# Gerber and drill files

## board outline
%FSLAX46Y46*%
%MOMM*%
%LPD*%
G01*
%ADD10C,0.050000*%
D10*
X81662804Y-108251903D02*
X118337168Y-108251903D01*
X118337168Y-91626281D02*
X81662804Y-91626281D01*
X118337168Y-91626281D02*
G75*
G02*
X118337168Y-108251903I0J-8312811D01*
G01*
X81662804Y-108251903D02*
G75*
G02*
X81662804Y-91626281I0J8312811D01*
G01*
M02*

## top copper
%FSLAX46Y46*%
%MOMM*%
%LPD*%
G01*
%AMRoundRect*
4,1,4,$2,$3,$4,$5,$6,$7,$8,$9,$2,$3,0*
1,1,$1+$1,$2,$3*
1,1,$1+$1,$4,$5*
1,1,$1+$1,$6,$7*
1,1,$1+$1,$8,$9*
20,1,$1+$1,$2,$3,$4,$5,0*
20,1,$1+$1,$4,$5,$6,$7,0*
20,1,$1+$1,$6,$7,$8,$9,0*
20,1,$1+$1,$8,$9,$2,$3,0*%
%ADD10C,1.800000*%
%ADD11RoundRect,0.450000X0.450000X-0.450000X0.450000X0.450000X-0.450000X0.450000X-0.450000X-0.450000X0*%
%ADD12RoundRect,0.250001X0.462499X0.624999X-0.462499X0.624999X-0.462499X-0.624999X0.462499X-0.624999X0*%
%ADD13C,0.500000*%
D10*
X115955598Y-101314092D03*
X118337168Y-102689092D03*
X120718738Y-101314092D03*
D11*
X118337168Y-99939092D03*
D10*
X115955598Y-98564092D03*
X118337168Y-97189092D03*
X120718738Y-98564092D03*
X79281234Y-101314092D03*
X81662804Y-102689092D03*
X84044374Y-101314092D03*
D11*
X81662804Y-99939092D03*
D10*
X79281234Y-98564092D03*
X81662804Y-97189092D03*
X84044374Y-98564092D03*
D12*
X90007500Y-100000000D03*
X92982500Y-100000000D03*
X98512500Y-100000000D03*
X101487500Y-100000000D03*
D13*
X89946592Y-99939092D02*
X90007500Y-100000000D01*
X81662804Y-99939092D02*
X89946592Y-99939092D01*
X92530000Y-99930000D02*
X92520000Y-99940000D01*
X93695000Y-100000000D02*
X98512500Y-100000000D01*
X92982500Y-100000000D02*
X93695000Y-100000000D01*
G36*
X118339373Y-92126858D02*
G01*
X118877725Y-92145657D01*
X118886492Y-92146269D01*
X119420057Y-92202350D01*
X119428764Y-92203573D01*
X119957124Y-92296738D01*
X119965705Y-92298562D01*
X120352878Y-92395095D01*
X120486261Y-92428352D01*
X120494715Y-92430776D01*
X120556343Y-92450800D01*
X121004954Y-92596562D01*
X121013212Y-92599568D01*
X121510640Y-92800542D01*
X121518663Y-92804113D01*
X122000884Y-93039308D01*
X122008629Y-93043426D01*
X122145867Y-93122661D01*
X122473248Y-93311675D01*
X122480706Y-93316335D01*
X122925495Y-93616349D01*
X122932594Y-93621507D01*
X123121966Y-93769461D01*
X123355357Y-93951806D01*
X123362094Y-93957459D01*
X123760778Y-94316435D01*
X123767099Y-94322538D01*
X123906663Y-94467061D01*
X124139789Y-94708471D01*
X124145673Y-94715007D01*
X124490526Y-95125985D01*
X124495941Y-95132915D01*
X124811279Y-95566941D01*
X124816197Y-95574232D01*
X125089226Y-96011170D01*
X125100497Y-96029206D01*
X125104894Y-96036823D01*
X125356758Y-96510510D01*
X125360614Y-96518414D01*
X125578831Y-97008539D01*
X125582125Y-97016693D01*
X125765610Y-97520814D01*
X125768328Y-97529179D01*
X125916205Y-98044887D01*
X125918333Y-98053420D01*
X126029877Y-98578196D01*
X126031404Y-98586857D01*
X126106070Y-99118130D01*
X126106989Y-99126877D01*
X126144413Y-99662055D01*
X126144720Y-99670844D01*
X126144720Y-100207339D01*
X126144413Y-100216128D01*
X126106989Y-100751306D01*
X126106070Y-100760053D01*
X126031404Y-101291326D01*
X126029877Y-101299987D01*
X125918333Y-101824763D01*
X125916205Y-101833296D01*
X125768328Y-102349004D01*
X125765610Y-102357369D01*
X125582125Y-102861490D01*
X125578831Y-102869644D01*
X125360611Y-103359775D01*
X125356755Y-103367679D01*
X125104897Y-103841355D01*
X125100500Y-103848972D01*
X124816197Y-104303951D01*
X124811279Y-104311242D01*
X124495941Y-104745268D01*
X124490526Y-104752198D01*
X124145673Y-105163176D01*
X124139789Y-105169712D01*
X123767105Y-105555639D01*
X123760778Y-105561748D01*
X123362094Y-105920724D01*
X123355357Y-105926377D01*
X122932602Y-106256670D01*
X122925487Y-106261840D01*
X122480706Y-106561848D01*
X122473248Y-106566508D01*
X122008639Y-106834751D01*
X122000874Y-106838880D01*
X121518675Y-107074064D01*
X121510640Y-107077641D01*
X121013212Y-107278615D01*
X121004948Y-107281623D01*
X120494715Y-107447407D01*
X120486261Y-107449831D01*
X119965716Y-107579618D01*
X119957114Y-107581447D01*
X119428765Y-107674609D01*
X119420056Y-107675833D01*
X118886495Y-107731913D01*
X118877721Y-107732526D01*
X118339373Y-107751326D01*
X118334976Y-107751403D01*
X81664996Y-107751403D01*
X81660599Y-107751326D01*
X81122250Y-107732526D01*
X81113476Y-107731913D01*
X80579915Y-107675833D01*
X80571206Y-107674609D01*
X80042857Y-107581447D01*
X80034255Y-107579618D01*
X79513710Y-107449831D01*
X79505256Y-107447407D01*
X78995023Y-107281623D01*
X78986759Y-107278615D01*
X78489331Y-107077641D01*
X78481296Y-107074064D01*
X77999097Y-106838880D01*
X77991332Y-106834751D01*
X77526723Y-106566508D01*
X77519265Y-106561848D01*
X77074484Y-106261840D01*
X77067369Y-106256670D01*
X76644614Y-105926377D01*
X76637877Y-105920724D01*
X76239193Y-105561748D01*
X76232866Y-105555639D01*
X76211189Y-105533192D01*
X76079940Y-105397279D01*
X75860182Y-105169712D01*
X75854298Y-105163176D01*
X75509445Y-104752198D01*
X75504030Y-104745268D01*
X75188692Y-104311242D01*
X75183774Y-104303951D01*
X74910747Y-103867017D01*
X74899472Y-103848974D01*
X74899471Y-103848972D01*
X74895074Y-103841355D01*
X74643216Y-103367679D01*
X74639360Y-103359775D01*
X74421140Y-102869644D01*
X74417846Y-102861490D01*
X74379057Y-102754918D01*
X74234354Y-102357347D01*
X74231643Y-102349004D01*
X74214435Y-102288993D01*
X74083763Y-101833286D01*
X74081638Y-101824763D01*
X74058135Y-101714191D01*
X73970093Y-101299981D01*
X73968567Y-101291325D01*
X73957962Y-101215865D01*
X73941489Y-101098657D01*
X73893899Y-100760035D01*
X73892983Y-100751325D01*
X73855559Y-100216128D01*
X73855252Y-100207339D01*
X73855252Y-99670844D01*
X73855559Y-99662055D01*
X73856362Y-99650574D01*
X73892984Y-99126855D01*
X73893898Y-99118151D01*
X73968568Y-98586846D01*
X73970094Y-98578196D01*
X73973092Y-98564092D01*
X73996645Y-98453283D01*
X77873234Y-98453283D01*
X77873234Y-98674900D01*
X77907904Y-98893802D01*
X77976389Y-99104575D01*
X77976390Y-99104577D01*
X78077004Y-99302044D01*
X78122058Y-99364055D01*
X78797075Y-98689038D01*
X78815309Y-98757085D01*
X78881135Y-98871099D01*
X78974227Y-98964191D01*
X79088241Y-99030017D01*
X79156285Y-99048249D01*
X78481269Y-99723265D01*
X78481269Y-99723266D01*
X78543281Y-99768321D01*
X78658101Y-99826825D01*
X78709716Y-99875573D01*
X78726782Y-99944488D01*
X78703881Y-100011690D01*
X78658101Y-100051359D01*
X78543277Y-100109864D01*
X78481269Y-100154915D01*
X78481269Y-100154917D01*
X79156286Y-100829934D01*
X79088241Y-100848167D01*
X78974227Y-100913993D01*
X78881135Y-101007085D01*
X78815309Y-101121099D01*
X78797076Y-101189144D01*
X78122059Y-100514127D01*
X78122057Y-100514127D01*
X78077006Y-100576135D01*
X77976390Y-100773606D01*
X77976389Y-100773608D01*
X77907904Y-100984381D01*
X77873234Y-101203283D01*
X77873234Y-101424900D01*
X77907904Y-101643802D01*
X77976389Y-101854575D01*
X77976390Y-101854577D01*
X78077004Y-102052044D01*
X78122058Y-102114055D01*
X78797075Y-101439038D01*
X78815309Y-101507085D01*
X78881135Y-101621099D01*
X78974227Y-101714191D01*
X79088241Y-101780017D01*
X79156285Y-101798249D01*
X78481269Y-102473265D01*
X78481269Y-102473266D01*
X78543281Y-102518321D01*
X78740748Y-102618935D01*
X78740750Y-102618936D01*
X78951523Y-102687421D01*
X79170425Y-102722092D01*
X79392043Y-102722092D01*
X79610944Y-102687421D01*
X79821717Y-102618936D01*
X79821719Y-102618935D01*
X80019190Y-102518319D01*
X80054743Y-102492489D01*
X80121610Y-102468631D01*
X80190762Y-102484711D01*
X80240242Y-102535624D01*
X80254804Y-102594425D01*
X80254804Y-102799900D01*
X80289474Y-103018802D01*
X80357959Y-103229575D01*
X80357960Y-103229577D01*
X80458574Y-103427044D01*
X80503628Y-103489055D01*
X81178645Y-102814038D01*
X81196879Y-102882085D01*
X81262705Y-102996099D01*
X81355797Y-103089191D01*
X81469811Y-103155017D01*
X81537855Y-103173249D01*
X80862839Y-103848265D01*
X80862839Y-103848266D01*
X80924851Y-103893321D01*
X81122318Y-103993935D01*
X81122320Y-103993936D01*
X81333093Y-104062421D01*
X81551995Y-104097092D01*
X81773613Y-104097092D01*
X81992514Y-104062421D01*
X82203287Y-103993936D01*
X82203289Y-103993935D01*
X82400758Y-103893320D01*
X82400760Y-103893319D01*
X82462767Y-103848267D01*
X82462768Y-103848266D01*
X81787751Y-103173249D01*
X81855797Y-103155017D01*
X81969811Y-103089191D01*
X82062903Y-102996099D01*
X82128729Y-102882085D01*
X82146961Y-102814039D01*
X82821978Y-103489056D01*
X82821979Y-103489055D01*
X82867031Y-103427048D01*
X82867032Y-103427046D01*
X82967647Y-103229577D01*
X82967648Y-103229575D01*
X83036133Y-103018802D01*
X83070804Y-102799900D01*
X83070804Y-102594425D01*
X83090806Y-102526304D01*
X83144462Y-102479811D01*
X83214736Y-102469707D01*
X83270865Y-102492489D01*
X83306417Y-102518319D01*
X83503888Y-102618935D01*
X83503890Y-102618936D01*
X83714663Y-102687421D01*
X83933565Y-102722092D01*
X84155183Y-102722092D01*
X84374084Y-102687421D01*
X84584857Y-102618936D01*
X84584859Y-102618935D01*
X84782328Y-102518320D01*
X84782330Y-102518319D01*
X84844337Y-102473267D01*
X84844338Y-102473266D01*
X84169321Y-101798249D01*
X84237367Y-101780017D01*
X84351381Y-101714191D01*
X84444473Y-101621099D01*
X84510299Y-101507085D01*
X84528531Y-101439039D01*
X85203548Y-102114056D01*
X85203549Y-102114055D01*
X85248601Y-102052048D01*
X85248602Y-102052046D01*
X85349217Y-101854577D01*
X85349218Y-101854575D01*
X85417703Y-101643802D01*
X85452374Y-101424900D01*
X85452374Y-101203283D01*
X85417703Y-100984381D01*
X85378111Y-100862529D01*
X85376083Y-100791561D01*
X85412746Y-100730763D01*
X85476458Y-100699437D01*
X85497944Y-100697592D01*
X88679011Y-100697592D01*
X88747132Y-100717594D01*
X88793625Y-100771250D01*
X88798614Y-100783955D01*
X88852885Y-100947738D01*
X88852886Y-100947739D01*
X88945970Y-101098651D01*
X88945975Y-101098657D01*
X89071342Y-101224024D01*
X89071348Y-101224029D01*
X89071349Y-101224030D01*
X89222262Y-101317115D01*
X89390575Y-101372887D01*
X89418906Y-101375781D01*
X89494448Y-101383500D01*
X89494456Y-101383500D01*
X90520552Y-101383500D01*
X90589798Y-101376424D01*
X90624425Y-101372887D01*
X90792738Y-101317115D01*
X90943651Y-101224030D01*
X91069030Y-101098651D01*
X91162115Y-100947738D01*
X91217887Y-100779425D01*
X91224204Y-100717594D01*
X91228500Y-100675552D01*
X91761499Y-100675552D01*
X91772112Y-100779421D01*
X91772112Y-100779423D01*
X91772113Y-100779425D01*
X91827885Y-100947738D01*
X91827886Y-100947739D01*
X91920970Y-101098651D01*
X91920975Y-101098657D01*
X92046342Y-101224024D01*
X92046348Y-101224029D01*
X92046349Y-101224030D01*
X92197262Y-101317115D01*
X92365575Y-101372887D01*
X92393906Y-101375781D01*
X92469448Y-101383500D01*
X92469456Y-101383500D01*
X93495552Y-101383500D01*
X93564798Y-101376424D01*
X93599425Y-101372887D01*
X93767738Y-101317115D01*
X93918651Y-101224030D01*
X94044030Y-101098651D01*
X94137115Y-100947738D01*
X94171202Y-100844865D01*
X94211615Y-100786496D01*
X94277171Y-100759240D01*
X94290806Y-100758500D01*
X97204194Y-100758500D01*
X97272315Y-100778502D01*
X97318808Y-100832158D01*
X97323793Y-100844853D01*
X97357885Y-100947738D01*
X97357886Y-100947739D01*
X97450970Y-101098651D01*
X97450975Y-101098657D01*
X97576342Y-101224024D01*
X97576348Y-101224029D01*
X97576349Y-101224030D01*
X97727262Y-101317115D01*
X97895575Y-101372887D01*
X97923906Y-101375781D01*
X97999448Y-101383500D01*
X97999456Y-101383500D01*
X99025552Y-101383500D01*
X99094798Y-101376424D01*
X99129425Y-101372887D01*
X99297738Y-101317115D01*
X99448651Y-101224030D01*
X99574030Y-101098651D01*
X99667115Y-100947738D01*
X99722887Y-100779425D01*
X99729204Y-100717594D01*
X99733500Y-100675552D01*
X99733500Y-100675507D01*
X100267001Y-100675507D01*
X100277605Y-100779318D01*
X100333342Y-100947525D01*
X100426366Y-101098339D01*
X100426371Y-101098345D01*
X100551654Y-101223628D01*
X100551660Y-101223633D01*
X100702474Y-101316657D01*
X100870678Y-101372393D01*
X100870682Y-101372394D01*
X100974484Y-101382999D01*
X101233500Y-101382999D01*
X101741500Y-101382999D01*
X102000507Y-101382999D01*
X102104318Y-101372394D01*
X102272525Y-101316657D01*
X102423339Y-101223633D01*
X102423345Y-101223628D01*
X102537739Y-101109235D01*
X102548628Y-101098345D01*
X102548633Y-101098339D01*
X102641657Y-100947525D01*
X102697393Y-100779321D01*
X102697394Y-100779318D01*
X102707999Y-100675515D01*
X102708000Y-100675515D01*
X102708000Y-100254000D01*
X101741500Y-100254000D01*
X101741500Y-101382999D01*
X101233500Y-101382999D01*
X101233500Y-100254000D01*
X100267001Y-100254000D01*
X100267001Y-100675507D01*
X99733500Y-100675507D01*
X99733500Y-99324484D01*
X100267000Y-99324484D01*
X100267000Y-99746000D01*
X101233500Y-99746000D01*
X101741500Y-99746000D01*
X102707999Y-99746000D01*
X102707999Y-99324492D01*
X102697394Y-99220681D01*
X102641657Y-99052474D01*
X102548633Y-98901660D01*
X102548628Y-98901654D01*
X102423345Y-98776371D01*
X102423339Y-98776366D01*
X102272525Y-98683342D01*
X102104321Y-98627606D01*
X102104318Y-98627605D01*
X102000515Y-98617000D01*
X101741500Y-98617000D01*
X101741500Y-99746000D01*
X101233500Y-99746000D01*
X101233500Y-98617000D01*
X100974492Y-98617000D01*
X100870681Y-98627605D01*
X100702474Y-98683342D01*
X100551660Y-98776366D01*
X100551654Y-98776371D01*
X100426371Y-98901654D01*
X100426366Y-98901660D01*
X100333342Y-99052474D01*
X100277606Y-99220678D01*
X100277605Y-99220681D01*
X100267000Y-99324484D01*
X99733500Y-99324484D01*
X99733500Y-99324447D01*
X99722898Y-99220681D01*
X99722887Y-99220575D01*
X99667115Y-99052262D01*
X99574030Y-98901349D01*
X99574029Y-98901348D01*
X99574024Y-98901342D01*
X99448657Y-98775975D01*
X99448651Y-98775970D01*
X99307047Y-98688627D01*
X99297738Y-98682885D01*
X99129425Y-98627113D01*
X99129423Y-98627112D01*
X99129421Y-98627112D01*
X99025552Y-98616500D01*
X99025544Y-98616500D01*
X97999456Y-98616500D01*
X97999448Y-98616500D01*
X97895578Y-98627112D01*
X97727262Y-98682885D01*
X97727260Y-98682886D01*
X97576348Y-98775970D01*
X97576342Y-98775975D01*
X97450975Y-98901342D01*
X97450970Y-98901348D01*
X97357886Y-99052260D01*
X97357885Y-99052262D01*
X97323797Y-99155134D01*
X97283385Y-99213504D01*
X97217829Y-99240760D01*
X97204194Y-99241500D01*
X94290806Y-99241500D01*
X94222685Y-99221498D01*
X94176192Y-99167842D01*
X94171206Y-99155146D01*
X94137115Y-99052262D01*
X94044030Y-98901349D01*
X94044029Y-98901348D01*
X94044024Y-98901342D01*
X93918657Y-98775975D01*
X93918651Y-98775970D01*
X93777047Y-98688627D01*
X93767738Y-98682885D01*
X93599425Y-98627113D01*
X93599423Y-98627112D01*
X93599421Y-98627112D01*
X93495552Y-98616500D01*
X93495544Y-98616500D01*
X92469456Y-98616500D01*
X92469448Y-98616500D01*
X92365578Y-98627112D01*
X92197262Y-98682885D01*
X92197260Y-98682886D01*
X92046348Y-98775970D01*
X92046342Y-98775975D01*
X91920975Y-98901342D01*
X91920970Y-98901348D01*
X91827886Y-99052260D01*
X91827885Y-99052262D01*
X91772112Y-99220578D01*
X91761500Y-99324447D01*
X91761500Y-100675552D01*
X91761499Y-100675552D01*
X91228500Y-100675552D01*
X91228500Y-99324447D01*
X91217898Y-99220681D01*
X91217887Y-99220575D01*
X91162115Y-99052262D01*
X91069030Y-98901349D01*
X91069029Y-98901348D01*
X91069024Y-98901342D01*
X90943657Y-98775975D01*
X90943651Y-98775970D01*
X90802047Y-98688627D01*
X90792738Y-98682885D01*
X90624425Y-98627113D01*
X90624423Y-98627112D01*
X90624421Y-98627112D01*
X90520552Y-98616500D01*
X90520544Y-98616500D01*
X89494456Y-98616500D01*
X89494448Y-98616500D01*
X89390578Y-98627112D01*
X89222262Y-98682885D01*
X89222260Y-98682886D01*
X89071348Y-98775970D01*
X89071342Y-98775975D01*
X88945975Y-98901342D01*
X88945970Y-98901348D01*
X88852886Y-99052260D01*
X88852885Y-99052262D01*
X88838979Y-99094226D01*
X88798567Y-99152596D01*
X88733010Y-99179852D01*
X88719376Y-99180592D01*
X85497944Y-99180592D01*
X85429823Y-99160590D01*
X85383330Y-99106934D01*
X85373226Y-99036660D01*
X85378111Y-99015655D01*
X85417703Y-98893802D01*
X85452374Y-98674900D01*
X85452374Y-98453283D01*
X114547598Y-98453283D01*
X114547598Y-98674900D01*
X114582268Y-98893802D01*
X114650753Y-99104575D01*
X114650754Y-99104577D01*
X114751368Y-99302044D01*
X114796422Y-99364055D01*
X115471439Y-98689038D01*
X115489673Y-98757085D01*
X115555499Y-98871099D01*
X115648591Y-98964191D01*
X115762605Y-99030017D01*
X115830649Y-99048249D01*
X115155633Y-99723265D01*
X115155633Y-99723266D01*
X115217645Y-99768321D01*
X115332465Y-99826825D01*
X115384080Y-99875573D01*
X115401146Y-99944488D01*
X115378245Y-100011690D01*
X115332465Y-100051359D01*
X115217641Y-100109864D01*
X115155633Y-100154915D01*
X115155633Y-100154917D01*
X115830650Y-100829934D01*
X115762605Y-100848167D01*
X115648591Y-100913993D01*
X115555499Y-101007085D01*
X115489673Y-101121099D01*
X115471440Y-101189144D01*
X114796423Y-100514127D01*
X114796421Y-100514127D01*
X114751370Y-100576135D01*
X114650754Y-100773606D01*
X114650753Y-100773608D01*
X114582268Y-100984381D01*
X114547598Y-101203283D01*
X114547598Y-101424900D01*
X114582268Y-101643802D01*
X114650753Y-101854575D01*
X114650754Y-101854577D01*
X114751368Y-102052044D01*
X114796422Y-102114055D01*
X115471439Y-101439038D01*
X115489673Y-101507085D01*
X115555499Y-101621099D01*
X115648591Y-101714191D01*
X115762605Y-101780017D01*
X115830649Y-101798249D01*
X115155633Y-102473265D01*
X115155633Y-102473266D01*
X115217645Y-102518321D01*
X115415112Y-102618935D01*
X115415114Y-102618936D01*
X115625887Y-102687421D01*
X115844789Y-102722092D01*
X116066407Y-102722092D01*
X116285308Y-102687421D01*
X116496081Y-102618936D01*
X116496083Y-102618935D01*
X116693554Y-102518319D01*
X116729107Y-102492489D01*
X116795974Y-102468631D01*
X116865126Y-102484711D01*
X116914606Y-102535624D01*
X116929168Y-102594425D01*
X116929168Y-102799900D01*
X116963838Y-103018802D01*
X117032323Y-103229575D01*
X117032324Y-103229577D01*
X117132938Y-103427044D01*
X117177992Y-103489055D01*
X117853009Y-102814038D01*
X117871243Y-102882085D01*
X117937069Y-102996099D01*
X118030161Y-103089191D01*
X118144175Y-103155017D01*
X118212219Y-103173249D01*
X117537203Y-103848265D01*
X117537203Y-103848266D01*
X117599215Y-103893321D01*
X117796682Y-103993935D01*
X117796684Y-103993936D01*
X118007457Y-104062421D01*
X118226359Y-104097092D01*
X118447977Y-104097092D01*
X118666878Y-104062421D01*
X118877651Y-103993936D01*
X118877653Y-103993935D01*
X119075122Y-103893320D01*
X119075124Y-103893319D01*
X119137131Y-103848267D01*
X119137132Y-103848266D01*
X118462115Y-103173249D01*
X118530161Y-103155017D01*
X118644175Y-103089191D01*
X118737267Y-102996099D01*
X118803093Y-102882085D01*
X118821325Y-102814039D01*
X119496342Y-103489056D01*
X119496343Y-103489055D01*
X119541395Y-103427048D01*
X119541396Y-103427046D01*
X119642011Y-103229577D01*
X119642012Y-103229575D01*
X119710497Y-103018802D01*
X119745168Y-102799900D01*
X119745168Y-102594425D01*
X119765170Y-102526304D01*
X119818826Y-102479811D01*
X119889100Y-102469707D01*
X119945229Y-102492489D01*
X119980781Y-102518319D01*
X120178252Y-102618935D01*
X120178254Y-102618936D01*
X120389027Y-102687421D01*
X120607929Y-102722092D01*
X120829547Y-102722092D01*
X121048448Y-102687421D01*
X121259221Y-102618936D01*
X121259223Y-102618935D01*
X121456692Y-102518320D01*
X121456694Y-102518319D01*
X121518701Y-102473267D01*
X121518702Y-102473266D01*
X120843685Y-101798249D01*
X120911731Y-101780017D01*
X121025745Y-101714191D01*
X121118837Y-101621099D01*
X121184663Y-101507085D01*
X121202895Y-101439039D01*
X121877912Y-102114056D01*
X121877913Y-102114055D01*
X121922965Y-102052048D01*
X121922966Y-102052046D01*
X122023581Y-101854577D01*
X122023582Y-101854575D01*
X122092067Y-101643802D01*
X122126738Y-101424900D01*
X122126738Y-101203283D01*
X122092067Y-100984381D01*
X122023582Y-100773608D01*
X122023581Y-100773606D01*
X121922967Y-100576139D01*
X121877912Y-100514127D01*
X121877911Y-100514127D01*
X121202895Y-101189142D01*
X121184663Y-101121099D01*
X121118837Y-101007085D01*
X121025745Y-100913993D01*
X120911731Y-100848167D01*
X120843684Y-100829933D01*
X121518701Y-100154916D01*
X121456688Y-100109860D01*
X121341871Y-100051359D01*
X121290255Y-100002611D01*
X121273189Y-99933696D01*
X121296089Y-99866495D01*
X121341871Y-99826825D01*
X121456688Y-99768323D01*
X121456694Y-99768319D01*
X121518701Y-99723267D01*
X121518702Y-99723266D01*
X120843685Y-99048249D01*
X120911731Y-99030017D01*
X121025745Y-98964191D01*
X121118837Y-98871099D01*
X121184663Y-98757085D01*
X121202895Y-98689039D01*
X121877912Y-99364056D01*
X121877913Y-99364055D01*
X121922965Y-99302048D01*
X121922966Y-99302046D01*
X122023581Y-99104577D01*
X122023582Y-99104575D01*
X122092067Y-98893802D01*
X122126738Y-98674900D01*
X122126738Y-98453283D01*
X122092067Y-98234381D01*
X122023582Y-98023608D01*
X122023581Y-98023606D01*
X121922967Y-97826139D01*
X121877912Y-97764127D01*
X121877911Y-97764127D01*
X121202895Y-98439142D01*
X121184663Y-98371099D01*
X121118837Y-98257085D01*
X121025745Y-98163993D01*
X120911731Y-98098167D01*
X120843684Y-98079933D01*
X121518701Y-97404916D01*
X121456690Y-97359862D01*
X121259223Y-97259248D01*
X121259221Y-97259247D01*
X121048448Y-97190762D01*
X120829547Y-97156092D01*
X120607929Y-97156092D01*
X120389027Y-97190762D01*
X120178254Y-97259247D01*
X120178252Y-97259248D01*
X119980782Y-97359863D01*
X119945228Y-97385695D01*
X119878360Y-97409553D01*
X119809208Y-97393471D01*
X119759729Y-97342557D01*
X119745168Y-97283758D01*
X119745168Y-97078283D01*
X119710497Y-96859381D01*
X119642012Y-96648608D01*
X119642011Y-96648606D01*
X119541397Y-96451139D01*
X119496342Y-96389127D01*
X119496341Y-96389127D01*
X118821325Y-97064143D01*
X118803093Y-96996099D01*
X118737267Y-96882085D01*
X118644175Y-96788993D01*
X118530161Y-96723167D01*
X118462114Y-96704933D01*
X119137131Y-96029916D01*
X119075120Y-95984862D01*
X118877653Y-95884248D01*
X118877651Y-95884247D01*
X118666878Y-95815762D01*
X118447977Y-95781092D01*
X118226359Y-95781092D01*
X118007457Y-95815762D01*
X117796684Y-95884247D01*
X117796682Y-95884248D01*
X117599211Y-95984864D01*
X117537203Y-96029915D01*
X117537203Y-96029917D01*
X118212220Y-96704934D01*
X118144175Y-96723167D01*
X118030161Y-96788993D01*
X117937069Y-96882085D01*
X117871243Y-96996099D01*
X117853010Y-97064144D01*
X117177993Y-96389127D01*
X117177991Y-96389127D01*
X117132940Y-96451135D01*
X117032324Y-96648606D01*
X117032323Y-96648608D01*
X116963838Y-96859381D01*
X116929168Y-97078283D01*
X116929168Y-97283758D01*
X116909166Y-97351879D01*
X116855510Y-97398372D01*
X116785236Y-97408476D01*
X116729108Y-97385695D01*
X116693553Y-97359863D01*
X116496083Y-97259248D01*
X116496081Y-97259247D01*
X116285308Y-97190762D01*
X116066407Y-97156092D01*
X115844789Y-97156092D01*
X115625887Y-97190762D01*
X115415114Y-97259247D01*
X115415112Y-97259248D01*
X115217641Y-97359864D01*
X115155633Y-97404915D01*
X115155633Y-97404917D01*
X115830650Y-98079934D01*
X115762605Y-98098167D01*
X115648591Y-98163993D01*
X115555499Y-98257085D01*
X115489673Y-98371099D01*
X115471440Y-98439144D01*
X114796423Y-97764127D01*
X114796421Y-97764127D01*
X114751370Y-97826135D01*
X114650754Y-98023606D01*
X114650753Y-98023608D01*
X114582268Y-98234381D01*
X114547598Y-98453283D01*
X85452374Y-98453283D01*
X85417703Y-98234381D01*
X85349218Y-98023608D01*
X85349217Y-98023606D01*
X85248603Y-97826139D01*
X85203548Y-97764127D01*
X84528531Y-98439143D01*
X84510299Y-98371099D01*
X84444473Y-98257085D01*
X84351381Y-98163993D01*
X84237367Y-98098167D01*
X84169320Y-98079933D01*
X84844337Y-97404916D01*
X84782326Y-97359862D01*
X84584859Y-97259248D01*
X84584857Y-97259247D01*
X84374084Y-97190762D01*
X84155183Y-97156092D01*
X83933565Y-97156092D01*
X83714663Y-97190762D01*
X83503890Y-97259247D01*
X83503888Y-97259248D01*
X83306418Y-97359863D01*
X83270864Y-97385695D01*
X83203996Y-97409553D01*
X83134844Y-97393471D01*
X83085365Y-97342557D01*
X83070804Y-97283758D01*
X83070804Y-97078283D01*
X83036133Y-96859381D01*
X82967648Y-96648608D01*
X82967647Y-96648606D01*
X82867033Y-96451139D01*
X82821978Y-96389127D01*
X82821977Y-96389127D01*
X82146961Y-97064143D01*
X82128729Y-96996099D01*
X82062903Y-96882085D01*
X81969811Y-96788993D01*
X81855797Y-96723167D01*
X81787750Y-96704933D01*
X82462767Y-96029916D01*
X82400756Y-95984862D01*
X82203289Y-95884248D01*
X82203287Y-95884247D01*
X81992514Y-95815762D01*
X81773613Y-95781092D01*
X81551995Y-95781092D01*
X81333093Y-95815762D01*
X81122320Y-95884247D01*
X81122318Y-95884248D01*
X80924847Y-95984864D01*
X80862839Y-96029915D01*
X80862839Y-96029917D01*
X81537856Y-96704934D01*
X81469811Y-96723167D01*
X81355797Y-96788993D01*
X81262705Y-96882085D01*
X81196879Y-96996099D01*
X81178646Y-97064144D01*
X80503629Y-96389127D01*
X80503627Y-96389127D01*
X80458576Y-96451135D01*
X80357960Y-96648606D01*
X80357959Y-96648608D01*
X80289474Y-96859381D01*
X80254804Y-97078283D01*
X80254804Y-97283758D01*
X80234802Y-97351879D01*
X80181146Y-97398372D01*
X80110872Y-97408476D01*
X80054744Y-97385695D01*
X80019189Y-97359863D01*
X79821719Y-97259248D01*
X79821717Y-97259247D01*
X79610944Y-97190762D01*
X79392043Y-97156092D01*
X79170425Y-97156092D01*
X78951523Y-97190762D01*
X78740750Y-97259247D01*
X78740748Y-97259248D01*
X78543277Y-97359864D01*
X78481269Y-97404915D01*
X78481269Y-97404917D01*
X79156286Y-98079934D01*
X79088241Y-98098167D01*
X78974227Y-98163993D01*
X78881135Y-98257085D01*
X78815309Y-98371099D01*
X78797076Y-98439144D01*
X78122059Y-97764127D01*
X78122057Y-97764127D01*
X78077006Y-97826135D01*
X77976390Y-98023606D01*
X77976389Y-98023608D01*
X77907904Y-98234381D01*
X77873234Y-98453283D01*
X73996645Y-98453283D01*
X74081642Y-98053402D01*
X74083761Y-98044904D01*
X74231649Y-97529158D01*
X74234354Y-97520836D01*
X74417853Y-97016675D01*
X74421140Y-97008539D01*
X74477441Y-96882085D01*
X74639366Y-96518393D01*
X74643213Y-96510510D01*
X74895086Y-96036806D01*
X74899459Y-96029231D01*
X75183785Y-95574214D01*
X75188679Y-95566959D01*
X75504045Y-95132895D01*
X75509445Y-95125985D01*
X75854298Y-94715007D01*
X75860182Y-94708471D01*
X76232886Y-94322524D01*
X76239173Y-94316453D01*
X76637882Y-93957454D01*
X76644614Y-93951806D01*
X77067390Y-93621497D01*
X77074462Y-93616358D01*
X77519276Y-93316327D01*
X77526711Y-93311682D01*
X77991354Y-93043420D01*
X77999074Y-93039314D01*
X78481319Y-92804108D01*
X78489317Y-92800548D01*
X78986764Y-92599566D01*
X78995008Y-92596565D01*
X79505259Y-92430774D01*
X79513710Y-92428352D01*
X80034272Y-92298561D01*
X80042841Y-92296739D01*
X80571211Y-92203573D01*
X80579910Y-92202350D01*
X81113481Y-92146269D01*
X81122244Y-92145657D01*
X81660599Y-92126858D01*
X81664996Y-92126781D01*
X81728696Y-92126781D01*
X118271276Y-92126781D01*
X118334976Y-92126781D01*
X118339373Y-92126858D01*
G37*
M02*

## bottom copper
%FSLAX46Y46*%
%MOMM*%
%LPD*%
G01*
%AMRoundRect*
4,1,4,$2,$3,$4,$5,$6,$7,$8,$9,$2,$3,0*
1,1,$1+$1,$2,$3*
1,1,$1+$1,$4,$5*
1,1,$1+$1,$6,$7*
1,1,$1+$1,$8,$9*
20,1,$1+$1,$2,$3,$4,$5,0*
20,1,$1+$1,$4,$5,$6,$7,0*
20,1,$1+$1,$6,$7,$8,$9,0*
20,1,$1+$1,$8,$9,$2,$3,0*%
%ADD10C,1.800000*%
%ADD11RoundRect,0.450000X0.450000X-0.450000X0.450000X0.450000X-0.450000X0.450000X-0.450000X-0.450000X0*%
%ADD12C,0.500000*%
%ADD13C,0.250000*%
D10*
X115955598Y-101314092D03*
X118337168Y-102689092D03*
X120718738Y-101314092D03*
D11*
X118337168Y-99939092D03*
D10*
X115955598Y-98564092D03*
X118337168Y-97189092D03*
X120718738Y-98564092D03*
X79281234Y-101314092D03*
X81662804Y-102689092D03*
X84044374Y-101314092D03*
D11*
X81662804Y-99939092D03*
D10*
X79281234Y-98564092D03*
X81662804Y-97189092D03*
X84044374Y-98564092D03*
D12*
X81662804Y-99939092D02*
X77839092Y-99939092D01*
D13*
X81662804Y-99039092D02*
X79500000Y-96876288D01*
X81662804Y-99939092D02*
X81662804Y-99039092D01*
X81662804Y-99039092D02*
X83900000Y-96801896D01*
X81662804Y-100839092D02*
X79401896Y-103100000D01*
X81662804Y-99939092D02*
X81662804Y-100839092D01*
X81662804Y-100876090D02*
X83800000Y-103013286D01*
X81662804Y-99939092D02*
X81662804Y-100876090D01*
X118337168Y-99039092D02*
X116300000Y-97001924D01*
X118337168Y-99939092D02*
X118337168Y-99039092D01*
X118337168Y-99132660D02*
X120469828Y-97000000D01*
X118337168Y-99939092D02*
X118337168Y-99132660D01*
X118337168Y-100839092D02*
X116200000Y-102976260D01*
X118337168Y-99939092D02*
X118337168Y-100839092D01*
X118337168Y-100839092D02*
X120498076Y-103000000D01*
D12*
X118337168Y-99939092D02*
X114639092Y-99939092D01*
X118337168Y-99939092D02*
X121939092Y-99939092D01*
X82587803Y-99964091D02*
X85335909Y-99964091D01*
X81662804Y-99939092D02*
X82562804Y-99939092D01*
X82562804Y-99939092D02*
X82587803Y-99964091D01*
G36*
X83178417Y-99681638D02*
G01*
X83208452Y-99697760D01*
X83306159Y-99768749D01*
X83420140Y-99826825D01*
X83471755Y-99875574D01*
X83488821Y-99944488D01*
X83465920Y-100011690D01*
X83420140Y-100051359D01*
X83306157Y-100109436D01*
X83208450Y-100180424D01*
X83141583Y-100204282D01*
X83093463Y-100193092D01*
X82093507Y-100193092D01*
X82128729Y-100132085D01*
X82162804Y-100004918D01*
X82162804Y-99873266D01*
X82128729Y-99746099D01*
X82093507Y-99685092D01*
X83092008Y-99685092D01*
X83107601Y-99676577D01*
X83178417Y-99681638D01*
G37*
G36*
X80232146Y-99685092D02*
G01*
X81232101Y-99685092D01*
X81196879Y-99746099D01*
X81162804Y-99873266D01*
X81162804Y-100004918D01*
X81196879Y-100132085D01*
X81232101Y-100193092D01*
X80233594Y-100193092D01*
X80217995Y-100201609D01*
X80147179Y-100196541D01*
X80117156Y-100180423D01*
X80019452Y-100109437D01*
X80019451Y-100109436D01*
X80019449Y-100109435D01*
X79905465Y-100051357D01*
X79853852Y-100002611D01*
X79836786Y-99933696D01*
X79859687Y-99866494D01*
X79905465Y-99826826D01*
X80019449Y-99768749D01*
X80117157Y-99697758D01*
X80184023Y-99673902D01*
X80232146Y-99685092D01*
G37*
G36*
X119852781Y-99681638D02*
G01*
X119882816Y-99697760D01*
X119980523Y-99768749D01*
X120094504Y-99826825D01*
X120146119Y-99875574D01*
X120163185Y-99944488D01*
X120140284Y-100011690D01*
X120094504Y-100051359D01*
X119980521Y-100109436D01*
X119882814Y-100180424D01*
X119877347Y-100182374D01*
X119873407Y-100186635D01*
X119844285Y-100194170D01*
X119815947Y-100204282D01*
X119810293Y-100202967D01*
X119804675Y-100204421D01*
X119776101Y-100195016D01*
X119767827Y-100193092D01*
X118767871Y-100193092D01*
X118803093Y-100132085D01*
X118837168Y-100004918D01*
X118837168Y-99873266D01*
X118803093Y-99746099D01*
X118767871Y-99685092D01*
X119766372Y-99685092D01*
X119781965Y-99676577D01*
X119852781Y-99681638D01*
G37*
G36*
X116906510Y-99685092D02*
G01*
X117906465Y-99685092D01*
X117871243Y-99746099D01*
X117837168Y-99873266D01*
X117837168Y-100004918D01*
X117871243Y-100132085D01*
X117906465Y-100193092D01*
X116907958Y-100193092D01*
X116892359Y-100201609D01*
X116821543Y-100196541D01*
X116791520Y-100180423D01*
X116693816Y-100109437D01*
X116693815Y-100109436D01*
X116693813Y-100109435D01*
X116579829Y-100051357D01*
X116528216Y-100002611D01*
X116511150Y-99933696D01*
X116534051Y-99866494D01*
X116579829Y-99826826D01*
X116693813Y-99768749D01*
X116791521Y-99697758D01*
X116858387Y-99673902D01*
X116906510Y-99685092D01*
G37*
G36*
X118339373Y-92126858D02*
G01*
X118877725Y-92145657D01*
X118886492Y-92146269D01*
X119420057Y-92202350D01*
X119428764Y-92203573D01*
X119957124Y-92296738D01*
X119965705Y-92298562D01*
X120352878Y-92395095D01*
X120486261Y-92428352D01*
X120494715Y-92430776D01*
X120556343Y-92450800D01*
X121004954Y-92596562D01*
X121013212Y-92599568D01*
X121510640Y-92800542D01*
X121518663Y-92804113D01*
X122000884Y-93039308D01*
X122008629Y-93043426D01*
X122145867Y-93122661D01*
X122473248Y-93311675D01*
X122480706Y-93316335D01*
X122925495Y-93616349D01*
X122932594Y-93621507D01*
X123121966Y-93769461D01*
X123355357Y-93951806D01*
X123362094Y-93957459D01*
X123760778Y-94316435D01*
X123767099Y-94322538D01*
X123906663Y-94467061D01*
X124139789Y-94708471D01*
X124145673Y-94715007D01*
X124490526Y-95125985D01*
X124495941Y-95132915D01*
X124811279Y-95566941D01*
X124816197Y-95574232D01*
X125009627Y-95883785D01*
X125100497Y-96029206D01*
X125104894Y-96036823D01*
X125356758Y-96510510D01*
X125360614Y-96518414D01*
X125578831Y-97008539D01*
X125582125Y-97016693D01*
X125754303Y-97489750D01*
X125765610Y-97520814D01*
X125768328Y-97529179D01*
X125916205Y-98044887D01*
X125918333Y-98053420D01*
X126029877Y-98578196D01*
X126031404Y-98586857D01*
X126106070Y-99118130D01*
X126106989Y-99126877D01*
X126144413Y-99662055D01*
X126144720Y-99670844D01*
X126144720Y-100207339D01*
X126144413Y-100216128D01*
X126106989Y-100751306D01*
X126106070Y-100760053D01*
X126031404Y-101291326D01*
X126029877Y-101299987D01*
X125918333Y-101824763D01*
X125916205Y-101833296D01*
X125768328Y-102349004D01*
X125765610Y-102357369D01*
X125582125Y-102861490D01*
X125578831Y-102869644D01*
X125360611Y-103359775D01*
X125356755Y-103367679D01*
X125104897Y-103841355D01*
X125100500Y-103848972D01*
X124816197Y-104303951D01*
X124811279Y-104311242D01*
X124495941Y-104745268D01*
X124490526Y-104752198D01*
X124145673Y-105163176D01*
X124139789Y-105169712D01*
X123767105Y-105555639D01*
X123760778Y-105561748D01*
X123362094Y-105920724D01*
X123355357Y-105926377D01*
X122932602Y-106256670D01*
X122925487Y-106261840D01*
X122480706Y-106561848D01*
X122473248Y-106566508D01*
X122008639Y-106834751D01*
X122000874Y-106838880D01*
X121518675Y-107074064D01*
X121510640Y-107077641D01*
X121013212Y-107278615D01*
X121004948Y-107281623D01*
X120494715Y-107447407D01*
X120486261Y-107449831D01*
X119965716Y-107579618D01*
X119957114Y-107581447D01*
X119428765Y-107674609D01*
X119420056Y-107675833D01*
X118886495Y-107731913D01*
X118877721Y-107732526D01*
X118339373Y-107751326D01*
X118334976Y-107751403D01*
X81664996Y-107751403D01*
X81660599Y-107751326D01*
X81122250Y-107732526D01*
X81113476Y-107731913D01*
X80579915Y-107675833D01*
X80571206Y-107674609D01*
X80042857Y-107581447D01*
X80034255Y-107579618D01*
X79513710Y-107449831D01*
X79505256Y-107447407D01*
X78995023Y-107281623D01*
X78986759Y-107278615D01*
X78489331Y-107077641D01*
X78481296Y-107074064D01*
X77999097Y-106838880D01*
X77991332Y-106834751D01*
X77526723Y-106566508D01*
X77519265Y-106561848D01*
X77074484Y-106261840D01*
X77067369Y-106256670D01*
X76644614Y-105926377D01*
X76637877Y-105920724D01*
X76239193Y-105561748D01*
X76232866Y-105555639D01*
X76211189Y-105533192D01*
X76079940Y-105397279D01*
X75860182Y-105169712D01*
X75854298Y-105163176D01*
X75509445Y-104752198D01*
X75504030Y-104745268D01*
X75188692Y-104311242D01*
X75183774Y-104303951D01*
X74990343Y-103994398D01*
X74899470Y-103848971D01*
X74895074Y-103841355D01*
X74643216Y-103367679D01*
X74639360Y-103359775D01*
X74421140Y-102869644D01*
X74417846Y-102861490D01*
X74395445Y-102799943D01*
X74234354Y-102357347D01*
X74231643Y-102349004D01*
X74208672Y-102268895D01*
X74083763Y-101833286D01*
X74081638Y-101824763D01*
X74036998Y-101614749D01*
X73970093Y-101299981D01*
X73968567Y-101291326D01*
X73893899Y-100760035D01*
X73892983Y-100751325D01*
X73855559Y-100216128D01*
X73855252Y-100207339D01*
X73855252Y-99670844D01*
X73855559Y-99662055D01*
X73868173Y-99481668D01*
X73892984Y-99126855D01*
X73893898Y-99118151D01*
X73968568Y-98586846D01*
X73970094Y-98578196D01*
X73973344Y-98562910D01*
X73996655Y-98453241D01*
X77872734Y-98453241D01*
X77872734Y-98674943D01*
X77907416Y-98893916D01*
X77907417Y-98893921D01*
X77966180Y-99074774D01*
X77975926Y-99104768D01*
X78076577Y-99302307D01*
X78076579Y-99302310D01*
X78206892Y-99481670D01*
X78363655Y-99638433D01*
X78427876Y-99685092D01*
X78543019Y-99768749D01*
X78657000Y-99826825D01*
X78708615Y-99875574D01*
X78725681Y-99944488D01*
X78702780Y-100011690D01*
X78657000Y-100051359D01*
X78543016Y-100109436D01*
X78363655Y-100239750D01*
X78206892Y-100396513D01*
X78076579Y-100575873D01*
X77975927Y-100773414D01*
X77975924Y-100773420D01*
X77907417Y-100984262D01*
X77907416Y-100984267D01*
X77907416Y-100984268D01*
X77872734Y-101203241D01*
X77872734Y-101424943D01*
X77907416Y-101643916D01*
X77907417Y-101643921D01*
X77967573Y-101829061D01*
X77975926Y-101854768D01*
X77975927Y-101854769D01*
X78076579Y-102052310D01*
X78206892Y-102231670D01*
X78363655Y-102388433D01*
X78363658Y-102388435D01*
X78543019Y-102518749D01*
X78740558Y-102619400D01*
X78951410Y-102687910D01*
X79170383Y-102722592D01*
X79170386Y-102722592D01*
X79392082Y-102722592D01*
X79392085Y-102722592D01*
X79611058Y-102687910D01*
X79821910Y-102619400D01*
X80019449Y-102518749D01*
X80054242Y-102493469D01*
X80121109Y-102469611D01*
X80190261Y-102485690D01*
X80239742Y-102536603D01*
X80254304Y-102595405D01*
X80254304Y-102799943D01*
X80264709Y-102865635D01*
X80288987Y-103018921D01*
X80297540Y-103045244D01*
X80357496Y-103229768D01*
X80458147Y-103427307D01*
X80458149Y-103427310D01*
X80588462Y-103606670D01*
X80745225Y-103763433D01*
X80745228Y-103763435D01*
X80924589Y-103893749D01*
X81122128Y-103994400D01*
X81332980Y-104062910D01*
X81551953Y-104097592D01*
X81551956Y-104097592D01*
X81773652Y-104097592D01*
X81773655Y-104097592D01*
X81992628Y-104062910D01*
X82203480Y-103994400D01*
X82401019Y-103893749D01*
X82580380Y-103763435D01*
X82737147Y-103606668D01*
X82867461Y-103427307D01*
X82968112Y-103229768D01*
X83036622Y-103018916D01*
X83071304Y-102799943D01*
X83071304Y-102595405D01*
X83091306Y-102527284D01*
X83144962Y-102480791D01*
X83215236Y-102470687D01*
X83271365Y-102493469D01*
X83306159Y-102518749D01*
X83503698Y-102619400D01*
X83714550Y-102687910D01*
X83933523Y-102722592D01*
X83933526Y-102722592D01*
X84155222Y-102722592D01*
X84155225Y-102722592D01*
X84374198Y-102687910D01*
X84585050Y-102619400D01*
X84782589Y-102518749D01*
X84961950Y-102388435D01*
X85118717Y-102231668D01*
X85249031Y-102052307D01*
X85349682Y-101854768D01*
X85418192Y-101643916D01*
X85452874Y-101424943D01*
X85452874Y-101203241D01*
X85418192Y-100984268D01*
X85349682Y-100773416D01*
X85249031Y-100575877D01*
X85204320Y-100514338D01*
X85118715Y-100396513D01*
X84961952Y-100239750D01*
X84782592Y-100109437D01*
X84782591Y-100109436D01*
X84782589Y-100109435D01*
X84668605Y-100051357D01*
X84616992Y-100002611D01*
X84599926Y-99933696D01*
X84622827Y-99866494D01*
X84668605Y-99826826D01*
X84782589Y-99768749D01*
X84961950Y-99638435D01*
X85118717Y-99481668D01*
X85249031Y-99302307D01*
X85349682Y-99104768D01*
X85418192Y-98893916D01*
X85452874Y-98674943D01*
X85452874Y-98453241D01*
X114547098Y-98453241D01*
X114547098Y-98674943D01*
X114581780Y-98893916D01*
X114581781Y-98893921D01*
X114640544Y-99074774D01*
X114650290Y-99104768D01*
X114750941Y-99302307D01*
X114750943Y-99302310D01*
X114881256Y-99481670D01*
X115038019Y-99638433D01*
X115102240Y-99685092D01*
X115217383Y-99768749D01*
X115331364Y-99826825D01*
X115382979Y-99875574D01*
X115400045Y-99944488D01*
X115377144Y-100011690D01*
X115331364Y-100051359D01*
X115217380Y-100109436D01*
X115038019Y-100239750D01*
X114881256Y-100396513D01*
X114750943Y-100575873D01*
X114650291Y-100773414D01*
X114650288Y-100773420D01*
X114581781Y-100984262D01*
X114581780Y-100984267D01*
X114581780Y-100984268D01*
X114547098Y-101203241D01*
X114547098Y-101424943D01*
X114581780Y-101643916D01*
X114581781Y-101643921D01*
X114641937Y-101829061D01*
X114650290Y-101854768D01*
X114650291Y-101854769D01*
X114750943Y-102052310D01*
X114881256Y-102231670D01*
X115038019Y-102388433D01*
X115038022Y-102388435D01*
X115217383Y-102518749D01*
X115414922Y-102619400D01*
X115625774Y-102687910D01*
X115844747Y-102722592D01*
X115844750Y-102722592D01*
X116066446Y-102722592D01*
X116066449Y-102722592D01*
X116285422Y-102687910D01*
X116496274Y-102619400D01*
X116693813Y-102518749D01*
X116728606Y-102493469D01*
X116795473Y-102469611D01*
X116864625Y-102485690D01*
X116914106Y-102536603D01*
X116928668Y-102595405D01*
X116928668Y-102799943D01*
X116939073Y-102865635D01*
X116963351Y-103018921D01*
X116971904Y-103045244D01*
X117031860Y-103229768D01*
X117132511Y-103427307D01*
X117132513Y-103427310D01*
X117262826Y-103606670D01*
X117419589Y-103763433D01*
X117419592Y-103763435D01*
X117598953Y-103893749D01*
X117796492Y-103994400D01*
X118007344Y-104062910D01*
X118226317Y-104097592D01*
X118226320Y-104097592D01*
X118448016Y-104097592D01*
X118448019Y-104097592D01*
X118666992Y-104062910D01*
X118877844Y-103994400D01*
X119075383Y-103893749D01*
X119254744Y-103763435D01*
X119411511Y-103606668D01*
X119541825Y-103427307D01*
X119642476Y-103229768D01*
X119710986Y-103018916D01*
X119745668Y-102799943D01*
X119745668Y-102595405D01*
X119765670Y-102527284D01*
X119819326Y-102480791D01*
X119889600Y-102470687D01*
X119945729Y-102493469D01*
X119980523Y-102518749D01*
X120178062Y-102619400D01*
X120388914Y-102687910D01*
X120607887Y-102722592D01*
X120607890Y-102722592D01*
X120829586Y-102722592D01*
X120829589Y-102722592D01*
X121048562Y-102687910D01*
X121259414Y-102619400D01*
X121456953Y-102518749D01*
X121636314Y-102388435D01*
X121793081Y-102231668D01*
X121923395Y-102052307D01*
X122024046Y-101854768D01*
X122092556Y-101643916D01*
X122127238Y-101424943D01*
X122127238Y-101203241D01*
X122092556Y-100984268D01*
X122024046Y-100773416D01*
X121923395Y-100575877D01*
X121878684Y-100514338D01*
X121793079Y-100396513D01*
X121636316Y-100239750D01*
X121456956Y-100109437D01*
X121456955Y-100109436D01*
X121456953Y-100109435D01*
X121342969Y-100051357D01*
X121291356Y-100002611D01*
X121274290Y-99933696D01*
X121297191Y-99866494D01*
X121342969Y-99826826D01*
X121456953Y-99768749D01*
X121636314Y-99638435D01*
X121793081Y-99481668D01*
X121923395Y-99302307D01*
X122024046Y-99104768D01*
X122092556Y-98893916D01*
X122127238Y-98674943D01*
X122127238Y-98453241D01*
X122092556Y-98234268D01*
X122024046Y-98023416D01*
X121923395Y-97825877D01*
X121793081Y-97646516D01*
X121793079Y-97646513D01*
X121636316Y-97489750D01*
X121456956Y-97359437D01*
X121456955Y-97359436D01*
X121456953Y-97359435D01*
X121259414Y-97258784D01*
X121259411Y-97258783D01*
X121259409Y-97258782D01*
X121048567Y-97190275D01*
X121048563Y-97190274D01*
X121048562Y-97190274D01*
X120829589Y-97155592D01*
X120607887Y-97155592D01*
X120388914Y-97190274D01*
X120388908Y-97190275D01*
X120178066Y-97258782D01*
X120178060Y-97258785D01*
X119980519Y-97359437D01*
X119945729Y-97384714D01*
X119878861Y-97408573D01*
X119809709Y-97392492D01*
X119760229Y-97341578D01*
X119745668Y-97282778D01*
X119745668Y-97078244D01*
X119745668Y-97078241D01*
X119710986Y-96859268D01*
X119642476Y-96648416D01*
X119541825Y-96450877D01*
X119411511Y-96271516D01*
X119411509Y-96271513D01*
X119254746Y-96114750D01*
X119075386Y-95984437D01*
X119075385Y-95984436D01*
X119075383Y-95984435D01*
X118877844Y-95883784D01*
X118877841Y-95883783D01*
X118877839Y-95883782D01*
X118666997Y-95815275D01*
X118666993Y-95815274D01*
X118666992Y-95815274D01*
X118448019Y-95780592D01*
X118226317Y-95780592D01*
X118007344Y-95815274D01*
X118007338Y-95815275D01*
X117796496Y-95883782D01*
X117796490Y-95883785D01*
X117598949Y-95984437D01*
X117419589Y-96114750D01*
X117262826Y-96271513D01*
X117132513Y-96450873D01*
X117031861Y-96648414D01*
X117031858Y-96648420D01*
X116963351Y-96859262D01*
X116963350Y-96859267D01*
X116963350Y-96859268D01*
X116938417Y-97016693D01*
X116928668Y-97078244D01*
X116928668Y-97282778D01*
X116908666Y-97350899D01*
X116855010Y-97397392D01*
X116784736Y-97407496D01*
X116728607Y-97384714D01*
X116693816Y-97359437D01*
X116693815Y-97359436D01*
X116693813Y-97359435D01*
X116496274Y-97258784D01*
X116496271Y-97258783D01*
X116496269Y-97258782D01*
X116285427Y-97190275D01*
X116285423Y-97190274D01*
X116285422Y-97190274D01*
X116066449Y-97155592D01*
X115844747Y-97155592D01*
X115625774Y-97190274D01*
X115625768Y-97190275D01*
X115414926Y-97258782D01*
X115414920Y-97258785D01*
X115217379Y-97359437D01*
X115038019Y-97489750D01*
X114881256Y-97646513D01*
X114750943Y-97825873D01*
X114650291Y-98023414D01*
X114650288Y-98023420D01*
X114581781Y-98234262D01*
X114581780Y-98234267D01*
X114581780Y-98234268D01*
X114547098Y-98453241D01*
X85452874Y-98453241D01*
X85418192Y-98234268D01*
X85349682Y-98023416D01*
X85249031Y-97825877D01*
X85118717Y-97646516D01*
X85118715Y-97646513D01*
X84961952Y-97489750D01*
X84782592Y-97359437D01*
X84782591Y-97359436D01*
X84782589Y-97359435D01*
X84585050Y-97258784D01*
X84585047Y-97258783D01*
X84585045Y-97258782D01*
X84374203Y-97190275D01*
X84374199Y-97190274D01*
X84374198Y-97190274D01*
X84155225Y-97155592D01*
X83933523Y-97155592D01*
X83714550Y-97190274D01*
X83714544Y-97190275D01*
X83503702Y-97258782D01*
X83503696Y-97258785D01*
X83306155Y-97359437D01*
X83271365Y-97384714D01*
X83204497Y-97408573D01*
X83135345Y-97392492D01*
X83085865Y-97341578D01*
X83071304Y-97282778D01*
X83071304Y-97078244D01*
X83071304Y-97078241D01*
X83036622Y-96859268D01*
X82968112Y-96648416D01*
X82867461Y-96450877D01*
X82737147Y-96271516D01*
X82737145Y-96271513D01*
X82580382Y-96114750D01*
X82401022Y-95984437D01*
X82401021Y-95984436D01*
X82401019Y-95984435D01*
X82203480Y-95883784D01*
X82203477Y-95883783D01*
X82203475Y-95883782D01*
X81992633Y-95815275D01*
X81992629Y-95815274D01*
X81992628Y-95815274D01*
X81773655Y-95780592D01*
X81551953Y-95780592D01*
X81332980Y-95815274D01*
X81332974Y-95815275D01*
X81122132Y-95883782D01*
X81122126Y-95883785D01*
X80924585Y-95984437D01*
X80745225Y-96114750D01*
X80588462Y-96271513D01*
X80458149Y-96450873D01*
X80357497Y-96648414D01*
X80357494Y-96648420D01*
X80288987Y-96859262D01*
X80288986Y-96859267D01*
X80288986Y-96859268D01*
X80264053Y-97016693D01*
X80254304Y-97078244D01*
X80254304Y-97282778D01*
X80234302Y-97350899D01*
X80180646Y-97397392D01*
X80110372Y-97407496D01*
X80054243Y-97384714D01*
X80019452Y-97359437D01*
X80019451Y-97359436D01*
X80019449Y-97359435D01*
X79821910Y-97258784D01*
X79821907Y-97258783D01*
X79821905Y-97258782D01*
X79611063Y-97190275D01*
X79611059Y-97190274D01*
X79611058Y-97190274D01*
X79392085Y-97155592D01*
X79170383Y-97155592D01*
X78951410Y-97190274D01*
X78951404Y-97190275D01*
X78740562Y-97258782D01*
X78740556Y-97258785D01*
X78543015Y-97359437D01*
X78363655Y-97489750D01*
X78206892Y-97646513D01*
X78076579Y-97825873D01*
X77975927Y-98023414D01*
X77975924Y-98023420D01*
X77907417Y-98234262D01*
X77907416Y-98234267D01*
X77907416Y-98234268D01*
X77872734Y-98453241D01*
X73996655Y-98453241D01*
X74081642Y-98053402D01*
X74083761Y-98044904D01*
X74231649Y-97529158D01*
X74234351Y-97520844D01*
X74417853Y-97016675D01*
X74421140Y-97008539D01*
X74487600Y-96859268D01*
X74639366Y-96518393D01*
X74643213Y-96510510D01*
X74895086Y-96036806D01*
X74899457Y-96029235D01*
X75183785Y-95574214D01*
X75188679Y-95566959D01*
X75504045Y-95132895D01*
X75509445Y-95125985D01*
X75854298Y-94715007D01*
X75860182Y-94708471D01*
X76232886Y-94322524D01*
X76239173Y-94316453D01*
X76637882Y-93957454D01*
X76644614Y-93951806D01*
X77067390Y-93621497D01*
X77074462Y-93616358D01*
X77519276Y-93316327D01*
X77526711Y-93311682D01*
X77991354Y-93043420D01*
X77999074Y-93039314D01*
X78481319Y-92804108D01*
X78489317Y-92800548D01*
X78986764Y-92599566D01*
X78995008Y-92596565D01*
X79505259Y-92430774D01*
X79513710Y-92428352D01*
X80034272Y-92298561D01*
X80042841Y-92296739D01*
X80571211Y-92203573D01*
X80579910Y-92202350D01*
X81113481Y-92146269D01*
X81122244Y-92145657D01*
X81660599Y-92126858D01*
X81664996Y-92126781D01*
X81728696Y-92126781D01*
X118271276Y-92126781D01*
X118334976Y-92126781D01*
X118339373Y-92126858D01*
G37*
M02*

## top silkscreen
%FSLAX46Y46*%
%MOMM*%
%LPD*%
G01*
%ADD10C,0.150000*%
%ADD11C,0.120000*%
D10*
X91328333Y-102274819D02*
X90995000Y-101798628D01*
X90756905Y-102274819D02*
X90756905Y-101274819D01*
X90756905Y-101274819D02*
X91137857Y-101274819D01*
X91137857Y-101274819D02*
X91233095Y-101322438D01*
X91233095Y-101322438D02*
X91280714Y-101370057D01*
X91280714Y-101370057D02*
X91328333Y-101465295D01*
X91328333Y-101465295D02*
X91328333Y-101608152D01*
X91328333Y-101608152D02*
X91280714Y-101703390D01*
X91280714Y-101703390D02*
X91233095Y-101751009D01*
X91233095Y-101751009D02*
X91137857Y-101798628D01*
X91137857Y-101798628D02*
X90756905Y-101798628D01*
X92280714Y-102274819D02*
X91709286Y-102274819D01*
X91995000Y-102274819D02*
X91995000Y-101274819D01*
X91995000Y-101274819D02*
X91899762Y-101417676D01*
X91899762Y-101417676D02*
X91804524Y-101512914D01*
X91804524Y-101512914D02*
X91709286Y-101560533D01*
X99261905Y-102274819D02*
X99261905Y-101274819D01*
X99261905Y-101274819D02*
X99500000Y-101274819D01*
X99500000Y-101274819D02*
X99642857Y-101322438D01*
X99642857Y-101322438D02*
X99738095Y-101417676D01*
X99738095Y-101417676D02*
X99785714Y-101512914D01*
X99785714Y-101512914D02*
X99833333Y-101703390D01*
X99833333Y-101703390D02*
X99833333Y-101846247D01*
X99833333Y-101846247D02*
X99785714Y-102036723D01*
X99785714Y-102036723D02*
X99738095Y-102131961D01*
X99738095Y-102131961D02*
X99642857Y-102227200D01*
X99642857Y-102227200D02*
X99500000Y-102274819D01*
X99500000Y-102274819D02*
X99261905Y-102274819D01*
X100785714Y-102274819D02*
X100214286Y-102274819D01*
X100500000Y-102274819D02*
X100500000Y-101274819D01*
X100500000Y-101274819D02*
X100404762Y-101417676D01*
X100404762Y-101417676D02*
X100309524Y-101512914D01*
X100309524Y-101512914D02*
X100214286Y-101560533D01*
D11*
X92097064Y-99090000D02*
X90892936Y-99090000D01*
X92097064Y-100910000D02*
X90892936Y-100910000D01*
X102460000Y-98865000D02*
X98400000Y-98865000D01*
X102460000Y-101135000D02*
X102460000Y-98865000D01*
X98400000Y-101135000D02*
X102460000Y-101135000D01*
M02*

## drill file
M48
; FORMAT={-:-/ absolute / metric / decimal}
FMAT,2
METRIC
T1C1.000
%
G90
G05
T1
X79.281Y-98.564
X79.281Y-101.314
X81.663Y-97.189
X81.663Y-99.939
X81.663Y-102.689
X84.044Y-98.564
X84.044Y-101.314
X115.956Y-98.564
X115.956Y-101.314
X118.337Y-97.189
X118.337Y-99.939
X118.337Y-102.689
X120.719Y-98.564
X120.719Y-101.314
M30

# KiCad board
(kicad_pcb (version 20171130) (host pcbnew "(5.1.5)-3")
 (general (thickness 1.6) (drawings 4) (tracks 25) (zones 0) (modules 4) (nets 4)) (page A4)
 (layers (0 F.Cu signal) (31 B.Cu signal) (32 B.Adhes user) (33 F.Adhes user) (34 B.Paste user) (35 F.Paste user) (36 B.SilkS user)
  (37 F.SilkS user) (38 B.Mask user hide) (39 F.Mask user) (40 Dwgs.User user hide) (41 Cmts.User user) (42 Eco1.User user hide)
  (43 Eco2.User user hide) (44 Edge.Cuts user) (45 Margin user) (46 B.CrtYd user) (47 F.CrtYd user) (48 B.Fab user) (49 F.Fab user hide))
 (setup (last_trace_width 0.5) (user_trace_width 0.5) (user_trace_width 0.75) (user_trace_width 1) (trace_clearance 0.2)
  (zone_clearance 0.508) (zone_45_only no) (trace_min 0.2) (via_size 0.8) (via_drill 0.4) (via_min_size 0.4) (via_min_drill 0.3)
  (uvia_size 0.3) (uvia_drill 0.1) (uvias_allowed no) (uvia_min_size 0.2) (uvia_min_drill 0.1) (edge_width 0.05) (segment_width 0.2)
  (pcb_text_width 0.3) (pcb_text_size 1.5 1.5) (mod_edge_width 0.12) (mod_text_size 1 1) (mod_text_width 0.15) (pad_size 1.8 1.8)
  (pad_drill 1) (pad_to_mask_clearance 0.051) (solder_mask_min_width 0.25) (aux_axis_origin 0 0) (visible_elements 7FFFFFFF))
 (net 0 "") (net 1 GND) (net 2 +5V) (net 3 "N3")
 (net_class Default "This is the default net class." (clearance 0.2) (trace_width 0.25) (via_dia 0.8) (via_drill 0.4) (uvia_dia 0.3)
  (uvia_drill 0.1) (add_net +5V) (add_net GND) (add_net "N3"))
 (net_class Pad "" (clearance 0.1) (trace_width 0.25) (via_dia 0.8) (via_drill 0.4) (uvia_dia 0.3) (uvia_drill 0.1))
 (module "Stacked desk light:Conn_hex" (layer F.Cu) (at 118.337168 99.939092 90)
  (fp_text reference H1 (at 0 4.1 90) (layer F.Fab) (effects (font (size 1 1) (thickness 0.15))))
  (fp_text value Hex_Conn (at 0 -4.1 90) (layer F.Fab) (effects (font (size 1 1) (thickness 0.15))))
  (pad 6 thru_hole circle (at -1.375 -2.38157 270) (size 1.8 1.8) (drill 1) (layers *.Cu *.Mask) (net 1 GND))
  (pad 5 thru_hole circle (at -2.75 0 270) (size 1.8 1.8) (drill 1) (layers *.Cu *.Mask) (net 1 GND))
  (pad 4 thru_hole circle (at -1.375 2.38157 270) (size 1.8 1.8) (drill 1) (layers *.Cu *.Mask) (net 1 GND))
  (pad 7 thru_hole roundrect (at 0 0 90) (size 1.8 1.8) (drill 1) (layers *.Cu *.Mask) (roundrect_rratio 0.25) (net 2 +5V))
  (pad 1 thru_hole circle (at 1.375 -2.38157 90) (size 1.8 1.8) (drill 1) (layers *.Cu *.Mask) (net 1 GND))
  (pad 2 thru_hole circle (at 2.75 0 90) (size 1.8 1.8) (drill 1) (layers *.Cu *.Mask) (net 1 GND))
  (pad 3 thru_hole circle (at 1.375 2.38157 90) (size 1.8 1.8) (drill 1) (layers *.Cu *.Mask) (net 1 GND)))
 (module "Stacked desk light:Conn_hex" (layer F.Cu) (at 81.662804 99.939092 90)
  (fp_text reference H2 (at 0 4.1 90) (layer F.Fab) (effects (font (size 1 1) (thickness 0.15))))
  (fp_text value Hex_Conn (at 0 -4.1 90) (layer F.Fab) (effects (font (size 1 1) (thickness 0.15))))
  (pad 6 thru_hole circle (at -1.375 -2.38157 270) (size 1.8 1.8) (drill 1) (layers *.Cu *.Mask) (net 1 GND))
  (pad 5 thru_hole circle (at -2.75 0 270) (size 1.8 1.8) (drill 1) (layers *.Cu *.Mask) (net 1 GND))
  (pad 4 thru_hole circle (at -1.375 2.38157 270) (size 1.8 1.8) (drill 1) (layers *.Cu *.Mask) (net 1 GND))
  (pad 7 thru_hole roundrect (at 0 0 90) (size 1.8 1.8) (drill 1) (layers *.Cu *.Mask) (roundrect_rratio 0.25) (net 2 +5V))
  (pad 1 thru_hole circle (at 1.375 -2.38157 90) (size 1.8 1.8) (drill 1) (layers *.Cu *.Mask) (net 1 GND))
  (pad 2 thru_hole circle (at 2.75 0 90) (size 1.8 1.8) (drill 1) (layers *.Cu *.Mask) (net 1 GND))
  (pad 3 thru_hole circle (at 1.375 2.38157 90) (size 1.8 1.8) (drill 1) (layers *.Cu *.Mask) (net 1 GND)))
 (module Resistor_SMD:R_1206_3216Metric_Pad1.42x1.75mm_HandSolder (layer F.Cu) (at 91.495 100 180)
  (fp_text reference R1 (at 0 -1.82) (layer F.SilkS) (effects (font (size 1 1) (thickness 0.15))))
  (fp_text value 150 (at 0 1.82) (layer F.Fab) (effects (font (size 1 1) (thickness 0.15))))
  (fp_line (start -0.602064 0.91) (end 0.602064 0.91) (layer F.SilkS) (width 0.12))
  (fp_line (start -0.602064 -0.91) (end 0.602064 -0.91) (layer F.SilkS) (width 0.12))
  (pad 2 smd roundrect (at 1.4875 0 180) (size 1.425 1.75) (layers F.Cu F.Paste F.Mask) (roundrect_rratio 0.175439) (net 2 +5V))
  (pad 1 smd roundrect (at -1.4875 0 180) (size 1.425 1.75) (layers F.Cu F.Paste F.Mask) (roundrect_rratio 0.175439) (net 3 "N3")))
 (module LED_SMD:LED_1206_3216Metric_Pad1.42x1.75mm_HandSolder (layer F.Cu) (at 100 100 180)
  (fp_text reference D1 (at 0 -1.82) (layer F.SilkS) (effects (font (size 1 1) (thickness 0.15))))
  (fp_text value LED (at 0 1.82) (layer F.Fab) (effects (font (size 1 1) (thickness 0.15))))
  (fp_line (start -2.46 1.135) (end 1.6 1.135) (layer F.SilkS) (width 0.12))
  (fp_line (start -2.46 -1.135) (end -2.46 1.135) (layer F.SilkS) (width 0.12))
  (fp_line (start 1.6 -1.135) (end -2.46 -1.135) (layer F.SilkS) (width 0.12))
  (pad 2 smd roundrect (at 1.4875 0 180) (size 1.425 1.75) (layers F.Cu F.Paste F.Mask) (roundrect_rratio 0.175439) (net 3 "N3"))
  (pad 1 smd roundrect (at -1.4875 0 180) (size 1.425 1.75) (layers F.Cu F.Paste F.Mask) (roundrect_rratio 0.175439) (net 1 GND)))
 (gr_line (start 81.662804 108.251903) (end 118.337168 108.251903) (layer Edge.Cuts) (width 0.05))
 (gr_line (start 118.337168 91.626281) (end 81.662804 91.626281) (layer Edge.Cuts) (width 0.05))
 (gr_arc (start 118.337168 99.939092) (end 118.337168 108.251903) (angle -180) (layer Edge.Cuts) (width 0.05))
 (gr_arc (start 81.662804 99.939092) (end 81.662804 91.626281) (angle -180) (layer Edge.Cuts) (width 0.05))
 (segment (start 89.946592 99.939092) (end 90.0075 100) (width 0.5) (layer F.Cu) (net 2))
 (segment (start 81.662804 99.939092) (end 89.946592 99.939092) (width 0.5) (layer F.Cu) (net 2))
 (segment (start 81.662804 99.939092) (end 77.839092 99.939092) (width 0.5) (layer B.Cu) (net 2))
 (segment (start 81.662804 99.039092) (end 79.5 96.876288) (width 0.25) (layer B.Cu) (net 2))
 (segment (start 81.662804 99.939092) (end 81.662804 99.039092) (width 0.25) (layer B.Cu) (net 2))
 (segment (start 81.662804 99.039092) (end 83.9 96.801896) (width 0.25) (layer B.Cu) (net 2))
 (segment (start 81.662804 100.839092) (end 79.401896 103.1) (width 0.25) (layer B.Cu) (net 2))
 (segment (start 81.662804 99.939092) (end 81.662804 100.839092) (width 0.25) (layer B.Cu) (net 2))
 (segment (start 81.662804 100.87609) (end 83.8 103.013286) (width 0.25) (layer B.Cu) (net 2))
 (segment (start 81.662804 99.939092) (end 81.662804 100.87609) (width 0.25) (layer B.Cu) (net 2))
 (segment (start 118.337168 99.039092) (end 116.3 97.001924) (width 0.25) (layer B.Cu) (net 2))
 (segment (start 118.337168 99.939092) (end 118.337168 99.039092) (width 0.25) (layer B.Cu) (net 2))
 (segment (start 118.337168 99.13266) (end 120.469828 97) (width 0.25) (layer B.Cu) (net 2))
 (segment (start 118.337168 99.939092) (end 118.337168 99.13266) (width 0.25) (layer B.Cu) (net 2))
 (segment (start 118.337168 100.839092) (end 116.2 102.97626) (width 0.25) (layer B.Cu) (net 2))
 (segment (start 118.337168 99.939092) (end 118.337168 100.839092) (width 0.25) (layer B.Cu) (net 2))
 (segment (start 118.337168 100.839092) (end 120.498076 103) (width 0.25) (layer B.Cu) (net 2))
 (segment (start 118.337168 99.939092) (end 114.639092 99.939092) (width 0.5) (layer B.Cu) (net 2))
 (segment (start 118.337168 99.939092) (end 121.939092 99.939092) (width 0.5) (layer B.Cu) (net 2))
 (segment (start 82.587803 99.964091) (end 85.335909 99.964091) (width 0.5) (layer B.Cu) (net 2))
 (segment (start 81.662804 99.939092) (end 82.562804 99.939092) (width 0.5) (layer B.Cu) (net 2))
 (segment (start 82.562804 99.939092) (end 82.587803 99.964091) (width 0.5) (layer B.Cu) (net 2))
 (segment (start 92.53 99.93) (end 92.52 99.94) (width 0.5) (layer F.Cu) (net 3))
 (segment (start 93.695 100) (end 98.5125 100) (width 0.5) (layer F.Cu) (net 3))
 (segment (start 92.9825 100) (end 93.695 100) (width 0.5) (layer F.Cu) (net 3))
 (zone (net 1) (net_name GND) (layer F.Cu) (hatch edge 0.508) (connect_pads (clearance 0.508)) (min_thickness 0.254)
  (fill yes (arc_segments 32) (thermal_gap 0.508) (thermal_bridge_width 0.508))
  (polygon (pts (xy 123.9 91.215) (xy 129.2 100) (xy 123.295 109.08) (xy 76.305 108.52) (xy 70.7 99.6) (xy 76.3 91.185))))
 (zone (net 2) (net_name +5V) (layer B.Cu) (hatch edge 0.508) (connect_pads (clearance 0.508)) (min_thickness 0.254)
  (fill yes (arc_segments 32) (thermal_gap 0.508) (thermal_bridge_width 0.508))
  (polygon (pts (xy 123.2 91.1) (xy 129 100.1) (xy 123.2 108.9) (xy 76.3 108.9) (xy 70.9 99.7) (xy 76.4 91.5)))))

